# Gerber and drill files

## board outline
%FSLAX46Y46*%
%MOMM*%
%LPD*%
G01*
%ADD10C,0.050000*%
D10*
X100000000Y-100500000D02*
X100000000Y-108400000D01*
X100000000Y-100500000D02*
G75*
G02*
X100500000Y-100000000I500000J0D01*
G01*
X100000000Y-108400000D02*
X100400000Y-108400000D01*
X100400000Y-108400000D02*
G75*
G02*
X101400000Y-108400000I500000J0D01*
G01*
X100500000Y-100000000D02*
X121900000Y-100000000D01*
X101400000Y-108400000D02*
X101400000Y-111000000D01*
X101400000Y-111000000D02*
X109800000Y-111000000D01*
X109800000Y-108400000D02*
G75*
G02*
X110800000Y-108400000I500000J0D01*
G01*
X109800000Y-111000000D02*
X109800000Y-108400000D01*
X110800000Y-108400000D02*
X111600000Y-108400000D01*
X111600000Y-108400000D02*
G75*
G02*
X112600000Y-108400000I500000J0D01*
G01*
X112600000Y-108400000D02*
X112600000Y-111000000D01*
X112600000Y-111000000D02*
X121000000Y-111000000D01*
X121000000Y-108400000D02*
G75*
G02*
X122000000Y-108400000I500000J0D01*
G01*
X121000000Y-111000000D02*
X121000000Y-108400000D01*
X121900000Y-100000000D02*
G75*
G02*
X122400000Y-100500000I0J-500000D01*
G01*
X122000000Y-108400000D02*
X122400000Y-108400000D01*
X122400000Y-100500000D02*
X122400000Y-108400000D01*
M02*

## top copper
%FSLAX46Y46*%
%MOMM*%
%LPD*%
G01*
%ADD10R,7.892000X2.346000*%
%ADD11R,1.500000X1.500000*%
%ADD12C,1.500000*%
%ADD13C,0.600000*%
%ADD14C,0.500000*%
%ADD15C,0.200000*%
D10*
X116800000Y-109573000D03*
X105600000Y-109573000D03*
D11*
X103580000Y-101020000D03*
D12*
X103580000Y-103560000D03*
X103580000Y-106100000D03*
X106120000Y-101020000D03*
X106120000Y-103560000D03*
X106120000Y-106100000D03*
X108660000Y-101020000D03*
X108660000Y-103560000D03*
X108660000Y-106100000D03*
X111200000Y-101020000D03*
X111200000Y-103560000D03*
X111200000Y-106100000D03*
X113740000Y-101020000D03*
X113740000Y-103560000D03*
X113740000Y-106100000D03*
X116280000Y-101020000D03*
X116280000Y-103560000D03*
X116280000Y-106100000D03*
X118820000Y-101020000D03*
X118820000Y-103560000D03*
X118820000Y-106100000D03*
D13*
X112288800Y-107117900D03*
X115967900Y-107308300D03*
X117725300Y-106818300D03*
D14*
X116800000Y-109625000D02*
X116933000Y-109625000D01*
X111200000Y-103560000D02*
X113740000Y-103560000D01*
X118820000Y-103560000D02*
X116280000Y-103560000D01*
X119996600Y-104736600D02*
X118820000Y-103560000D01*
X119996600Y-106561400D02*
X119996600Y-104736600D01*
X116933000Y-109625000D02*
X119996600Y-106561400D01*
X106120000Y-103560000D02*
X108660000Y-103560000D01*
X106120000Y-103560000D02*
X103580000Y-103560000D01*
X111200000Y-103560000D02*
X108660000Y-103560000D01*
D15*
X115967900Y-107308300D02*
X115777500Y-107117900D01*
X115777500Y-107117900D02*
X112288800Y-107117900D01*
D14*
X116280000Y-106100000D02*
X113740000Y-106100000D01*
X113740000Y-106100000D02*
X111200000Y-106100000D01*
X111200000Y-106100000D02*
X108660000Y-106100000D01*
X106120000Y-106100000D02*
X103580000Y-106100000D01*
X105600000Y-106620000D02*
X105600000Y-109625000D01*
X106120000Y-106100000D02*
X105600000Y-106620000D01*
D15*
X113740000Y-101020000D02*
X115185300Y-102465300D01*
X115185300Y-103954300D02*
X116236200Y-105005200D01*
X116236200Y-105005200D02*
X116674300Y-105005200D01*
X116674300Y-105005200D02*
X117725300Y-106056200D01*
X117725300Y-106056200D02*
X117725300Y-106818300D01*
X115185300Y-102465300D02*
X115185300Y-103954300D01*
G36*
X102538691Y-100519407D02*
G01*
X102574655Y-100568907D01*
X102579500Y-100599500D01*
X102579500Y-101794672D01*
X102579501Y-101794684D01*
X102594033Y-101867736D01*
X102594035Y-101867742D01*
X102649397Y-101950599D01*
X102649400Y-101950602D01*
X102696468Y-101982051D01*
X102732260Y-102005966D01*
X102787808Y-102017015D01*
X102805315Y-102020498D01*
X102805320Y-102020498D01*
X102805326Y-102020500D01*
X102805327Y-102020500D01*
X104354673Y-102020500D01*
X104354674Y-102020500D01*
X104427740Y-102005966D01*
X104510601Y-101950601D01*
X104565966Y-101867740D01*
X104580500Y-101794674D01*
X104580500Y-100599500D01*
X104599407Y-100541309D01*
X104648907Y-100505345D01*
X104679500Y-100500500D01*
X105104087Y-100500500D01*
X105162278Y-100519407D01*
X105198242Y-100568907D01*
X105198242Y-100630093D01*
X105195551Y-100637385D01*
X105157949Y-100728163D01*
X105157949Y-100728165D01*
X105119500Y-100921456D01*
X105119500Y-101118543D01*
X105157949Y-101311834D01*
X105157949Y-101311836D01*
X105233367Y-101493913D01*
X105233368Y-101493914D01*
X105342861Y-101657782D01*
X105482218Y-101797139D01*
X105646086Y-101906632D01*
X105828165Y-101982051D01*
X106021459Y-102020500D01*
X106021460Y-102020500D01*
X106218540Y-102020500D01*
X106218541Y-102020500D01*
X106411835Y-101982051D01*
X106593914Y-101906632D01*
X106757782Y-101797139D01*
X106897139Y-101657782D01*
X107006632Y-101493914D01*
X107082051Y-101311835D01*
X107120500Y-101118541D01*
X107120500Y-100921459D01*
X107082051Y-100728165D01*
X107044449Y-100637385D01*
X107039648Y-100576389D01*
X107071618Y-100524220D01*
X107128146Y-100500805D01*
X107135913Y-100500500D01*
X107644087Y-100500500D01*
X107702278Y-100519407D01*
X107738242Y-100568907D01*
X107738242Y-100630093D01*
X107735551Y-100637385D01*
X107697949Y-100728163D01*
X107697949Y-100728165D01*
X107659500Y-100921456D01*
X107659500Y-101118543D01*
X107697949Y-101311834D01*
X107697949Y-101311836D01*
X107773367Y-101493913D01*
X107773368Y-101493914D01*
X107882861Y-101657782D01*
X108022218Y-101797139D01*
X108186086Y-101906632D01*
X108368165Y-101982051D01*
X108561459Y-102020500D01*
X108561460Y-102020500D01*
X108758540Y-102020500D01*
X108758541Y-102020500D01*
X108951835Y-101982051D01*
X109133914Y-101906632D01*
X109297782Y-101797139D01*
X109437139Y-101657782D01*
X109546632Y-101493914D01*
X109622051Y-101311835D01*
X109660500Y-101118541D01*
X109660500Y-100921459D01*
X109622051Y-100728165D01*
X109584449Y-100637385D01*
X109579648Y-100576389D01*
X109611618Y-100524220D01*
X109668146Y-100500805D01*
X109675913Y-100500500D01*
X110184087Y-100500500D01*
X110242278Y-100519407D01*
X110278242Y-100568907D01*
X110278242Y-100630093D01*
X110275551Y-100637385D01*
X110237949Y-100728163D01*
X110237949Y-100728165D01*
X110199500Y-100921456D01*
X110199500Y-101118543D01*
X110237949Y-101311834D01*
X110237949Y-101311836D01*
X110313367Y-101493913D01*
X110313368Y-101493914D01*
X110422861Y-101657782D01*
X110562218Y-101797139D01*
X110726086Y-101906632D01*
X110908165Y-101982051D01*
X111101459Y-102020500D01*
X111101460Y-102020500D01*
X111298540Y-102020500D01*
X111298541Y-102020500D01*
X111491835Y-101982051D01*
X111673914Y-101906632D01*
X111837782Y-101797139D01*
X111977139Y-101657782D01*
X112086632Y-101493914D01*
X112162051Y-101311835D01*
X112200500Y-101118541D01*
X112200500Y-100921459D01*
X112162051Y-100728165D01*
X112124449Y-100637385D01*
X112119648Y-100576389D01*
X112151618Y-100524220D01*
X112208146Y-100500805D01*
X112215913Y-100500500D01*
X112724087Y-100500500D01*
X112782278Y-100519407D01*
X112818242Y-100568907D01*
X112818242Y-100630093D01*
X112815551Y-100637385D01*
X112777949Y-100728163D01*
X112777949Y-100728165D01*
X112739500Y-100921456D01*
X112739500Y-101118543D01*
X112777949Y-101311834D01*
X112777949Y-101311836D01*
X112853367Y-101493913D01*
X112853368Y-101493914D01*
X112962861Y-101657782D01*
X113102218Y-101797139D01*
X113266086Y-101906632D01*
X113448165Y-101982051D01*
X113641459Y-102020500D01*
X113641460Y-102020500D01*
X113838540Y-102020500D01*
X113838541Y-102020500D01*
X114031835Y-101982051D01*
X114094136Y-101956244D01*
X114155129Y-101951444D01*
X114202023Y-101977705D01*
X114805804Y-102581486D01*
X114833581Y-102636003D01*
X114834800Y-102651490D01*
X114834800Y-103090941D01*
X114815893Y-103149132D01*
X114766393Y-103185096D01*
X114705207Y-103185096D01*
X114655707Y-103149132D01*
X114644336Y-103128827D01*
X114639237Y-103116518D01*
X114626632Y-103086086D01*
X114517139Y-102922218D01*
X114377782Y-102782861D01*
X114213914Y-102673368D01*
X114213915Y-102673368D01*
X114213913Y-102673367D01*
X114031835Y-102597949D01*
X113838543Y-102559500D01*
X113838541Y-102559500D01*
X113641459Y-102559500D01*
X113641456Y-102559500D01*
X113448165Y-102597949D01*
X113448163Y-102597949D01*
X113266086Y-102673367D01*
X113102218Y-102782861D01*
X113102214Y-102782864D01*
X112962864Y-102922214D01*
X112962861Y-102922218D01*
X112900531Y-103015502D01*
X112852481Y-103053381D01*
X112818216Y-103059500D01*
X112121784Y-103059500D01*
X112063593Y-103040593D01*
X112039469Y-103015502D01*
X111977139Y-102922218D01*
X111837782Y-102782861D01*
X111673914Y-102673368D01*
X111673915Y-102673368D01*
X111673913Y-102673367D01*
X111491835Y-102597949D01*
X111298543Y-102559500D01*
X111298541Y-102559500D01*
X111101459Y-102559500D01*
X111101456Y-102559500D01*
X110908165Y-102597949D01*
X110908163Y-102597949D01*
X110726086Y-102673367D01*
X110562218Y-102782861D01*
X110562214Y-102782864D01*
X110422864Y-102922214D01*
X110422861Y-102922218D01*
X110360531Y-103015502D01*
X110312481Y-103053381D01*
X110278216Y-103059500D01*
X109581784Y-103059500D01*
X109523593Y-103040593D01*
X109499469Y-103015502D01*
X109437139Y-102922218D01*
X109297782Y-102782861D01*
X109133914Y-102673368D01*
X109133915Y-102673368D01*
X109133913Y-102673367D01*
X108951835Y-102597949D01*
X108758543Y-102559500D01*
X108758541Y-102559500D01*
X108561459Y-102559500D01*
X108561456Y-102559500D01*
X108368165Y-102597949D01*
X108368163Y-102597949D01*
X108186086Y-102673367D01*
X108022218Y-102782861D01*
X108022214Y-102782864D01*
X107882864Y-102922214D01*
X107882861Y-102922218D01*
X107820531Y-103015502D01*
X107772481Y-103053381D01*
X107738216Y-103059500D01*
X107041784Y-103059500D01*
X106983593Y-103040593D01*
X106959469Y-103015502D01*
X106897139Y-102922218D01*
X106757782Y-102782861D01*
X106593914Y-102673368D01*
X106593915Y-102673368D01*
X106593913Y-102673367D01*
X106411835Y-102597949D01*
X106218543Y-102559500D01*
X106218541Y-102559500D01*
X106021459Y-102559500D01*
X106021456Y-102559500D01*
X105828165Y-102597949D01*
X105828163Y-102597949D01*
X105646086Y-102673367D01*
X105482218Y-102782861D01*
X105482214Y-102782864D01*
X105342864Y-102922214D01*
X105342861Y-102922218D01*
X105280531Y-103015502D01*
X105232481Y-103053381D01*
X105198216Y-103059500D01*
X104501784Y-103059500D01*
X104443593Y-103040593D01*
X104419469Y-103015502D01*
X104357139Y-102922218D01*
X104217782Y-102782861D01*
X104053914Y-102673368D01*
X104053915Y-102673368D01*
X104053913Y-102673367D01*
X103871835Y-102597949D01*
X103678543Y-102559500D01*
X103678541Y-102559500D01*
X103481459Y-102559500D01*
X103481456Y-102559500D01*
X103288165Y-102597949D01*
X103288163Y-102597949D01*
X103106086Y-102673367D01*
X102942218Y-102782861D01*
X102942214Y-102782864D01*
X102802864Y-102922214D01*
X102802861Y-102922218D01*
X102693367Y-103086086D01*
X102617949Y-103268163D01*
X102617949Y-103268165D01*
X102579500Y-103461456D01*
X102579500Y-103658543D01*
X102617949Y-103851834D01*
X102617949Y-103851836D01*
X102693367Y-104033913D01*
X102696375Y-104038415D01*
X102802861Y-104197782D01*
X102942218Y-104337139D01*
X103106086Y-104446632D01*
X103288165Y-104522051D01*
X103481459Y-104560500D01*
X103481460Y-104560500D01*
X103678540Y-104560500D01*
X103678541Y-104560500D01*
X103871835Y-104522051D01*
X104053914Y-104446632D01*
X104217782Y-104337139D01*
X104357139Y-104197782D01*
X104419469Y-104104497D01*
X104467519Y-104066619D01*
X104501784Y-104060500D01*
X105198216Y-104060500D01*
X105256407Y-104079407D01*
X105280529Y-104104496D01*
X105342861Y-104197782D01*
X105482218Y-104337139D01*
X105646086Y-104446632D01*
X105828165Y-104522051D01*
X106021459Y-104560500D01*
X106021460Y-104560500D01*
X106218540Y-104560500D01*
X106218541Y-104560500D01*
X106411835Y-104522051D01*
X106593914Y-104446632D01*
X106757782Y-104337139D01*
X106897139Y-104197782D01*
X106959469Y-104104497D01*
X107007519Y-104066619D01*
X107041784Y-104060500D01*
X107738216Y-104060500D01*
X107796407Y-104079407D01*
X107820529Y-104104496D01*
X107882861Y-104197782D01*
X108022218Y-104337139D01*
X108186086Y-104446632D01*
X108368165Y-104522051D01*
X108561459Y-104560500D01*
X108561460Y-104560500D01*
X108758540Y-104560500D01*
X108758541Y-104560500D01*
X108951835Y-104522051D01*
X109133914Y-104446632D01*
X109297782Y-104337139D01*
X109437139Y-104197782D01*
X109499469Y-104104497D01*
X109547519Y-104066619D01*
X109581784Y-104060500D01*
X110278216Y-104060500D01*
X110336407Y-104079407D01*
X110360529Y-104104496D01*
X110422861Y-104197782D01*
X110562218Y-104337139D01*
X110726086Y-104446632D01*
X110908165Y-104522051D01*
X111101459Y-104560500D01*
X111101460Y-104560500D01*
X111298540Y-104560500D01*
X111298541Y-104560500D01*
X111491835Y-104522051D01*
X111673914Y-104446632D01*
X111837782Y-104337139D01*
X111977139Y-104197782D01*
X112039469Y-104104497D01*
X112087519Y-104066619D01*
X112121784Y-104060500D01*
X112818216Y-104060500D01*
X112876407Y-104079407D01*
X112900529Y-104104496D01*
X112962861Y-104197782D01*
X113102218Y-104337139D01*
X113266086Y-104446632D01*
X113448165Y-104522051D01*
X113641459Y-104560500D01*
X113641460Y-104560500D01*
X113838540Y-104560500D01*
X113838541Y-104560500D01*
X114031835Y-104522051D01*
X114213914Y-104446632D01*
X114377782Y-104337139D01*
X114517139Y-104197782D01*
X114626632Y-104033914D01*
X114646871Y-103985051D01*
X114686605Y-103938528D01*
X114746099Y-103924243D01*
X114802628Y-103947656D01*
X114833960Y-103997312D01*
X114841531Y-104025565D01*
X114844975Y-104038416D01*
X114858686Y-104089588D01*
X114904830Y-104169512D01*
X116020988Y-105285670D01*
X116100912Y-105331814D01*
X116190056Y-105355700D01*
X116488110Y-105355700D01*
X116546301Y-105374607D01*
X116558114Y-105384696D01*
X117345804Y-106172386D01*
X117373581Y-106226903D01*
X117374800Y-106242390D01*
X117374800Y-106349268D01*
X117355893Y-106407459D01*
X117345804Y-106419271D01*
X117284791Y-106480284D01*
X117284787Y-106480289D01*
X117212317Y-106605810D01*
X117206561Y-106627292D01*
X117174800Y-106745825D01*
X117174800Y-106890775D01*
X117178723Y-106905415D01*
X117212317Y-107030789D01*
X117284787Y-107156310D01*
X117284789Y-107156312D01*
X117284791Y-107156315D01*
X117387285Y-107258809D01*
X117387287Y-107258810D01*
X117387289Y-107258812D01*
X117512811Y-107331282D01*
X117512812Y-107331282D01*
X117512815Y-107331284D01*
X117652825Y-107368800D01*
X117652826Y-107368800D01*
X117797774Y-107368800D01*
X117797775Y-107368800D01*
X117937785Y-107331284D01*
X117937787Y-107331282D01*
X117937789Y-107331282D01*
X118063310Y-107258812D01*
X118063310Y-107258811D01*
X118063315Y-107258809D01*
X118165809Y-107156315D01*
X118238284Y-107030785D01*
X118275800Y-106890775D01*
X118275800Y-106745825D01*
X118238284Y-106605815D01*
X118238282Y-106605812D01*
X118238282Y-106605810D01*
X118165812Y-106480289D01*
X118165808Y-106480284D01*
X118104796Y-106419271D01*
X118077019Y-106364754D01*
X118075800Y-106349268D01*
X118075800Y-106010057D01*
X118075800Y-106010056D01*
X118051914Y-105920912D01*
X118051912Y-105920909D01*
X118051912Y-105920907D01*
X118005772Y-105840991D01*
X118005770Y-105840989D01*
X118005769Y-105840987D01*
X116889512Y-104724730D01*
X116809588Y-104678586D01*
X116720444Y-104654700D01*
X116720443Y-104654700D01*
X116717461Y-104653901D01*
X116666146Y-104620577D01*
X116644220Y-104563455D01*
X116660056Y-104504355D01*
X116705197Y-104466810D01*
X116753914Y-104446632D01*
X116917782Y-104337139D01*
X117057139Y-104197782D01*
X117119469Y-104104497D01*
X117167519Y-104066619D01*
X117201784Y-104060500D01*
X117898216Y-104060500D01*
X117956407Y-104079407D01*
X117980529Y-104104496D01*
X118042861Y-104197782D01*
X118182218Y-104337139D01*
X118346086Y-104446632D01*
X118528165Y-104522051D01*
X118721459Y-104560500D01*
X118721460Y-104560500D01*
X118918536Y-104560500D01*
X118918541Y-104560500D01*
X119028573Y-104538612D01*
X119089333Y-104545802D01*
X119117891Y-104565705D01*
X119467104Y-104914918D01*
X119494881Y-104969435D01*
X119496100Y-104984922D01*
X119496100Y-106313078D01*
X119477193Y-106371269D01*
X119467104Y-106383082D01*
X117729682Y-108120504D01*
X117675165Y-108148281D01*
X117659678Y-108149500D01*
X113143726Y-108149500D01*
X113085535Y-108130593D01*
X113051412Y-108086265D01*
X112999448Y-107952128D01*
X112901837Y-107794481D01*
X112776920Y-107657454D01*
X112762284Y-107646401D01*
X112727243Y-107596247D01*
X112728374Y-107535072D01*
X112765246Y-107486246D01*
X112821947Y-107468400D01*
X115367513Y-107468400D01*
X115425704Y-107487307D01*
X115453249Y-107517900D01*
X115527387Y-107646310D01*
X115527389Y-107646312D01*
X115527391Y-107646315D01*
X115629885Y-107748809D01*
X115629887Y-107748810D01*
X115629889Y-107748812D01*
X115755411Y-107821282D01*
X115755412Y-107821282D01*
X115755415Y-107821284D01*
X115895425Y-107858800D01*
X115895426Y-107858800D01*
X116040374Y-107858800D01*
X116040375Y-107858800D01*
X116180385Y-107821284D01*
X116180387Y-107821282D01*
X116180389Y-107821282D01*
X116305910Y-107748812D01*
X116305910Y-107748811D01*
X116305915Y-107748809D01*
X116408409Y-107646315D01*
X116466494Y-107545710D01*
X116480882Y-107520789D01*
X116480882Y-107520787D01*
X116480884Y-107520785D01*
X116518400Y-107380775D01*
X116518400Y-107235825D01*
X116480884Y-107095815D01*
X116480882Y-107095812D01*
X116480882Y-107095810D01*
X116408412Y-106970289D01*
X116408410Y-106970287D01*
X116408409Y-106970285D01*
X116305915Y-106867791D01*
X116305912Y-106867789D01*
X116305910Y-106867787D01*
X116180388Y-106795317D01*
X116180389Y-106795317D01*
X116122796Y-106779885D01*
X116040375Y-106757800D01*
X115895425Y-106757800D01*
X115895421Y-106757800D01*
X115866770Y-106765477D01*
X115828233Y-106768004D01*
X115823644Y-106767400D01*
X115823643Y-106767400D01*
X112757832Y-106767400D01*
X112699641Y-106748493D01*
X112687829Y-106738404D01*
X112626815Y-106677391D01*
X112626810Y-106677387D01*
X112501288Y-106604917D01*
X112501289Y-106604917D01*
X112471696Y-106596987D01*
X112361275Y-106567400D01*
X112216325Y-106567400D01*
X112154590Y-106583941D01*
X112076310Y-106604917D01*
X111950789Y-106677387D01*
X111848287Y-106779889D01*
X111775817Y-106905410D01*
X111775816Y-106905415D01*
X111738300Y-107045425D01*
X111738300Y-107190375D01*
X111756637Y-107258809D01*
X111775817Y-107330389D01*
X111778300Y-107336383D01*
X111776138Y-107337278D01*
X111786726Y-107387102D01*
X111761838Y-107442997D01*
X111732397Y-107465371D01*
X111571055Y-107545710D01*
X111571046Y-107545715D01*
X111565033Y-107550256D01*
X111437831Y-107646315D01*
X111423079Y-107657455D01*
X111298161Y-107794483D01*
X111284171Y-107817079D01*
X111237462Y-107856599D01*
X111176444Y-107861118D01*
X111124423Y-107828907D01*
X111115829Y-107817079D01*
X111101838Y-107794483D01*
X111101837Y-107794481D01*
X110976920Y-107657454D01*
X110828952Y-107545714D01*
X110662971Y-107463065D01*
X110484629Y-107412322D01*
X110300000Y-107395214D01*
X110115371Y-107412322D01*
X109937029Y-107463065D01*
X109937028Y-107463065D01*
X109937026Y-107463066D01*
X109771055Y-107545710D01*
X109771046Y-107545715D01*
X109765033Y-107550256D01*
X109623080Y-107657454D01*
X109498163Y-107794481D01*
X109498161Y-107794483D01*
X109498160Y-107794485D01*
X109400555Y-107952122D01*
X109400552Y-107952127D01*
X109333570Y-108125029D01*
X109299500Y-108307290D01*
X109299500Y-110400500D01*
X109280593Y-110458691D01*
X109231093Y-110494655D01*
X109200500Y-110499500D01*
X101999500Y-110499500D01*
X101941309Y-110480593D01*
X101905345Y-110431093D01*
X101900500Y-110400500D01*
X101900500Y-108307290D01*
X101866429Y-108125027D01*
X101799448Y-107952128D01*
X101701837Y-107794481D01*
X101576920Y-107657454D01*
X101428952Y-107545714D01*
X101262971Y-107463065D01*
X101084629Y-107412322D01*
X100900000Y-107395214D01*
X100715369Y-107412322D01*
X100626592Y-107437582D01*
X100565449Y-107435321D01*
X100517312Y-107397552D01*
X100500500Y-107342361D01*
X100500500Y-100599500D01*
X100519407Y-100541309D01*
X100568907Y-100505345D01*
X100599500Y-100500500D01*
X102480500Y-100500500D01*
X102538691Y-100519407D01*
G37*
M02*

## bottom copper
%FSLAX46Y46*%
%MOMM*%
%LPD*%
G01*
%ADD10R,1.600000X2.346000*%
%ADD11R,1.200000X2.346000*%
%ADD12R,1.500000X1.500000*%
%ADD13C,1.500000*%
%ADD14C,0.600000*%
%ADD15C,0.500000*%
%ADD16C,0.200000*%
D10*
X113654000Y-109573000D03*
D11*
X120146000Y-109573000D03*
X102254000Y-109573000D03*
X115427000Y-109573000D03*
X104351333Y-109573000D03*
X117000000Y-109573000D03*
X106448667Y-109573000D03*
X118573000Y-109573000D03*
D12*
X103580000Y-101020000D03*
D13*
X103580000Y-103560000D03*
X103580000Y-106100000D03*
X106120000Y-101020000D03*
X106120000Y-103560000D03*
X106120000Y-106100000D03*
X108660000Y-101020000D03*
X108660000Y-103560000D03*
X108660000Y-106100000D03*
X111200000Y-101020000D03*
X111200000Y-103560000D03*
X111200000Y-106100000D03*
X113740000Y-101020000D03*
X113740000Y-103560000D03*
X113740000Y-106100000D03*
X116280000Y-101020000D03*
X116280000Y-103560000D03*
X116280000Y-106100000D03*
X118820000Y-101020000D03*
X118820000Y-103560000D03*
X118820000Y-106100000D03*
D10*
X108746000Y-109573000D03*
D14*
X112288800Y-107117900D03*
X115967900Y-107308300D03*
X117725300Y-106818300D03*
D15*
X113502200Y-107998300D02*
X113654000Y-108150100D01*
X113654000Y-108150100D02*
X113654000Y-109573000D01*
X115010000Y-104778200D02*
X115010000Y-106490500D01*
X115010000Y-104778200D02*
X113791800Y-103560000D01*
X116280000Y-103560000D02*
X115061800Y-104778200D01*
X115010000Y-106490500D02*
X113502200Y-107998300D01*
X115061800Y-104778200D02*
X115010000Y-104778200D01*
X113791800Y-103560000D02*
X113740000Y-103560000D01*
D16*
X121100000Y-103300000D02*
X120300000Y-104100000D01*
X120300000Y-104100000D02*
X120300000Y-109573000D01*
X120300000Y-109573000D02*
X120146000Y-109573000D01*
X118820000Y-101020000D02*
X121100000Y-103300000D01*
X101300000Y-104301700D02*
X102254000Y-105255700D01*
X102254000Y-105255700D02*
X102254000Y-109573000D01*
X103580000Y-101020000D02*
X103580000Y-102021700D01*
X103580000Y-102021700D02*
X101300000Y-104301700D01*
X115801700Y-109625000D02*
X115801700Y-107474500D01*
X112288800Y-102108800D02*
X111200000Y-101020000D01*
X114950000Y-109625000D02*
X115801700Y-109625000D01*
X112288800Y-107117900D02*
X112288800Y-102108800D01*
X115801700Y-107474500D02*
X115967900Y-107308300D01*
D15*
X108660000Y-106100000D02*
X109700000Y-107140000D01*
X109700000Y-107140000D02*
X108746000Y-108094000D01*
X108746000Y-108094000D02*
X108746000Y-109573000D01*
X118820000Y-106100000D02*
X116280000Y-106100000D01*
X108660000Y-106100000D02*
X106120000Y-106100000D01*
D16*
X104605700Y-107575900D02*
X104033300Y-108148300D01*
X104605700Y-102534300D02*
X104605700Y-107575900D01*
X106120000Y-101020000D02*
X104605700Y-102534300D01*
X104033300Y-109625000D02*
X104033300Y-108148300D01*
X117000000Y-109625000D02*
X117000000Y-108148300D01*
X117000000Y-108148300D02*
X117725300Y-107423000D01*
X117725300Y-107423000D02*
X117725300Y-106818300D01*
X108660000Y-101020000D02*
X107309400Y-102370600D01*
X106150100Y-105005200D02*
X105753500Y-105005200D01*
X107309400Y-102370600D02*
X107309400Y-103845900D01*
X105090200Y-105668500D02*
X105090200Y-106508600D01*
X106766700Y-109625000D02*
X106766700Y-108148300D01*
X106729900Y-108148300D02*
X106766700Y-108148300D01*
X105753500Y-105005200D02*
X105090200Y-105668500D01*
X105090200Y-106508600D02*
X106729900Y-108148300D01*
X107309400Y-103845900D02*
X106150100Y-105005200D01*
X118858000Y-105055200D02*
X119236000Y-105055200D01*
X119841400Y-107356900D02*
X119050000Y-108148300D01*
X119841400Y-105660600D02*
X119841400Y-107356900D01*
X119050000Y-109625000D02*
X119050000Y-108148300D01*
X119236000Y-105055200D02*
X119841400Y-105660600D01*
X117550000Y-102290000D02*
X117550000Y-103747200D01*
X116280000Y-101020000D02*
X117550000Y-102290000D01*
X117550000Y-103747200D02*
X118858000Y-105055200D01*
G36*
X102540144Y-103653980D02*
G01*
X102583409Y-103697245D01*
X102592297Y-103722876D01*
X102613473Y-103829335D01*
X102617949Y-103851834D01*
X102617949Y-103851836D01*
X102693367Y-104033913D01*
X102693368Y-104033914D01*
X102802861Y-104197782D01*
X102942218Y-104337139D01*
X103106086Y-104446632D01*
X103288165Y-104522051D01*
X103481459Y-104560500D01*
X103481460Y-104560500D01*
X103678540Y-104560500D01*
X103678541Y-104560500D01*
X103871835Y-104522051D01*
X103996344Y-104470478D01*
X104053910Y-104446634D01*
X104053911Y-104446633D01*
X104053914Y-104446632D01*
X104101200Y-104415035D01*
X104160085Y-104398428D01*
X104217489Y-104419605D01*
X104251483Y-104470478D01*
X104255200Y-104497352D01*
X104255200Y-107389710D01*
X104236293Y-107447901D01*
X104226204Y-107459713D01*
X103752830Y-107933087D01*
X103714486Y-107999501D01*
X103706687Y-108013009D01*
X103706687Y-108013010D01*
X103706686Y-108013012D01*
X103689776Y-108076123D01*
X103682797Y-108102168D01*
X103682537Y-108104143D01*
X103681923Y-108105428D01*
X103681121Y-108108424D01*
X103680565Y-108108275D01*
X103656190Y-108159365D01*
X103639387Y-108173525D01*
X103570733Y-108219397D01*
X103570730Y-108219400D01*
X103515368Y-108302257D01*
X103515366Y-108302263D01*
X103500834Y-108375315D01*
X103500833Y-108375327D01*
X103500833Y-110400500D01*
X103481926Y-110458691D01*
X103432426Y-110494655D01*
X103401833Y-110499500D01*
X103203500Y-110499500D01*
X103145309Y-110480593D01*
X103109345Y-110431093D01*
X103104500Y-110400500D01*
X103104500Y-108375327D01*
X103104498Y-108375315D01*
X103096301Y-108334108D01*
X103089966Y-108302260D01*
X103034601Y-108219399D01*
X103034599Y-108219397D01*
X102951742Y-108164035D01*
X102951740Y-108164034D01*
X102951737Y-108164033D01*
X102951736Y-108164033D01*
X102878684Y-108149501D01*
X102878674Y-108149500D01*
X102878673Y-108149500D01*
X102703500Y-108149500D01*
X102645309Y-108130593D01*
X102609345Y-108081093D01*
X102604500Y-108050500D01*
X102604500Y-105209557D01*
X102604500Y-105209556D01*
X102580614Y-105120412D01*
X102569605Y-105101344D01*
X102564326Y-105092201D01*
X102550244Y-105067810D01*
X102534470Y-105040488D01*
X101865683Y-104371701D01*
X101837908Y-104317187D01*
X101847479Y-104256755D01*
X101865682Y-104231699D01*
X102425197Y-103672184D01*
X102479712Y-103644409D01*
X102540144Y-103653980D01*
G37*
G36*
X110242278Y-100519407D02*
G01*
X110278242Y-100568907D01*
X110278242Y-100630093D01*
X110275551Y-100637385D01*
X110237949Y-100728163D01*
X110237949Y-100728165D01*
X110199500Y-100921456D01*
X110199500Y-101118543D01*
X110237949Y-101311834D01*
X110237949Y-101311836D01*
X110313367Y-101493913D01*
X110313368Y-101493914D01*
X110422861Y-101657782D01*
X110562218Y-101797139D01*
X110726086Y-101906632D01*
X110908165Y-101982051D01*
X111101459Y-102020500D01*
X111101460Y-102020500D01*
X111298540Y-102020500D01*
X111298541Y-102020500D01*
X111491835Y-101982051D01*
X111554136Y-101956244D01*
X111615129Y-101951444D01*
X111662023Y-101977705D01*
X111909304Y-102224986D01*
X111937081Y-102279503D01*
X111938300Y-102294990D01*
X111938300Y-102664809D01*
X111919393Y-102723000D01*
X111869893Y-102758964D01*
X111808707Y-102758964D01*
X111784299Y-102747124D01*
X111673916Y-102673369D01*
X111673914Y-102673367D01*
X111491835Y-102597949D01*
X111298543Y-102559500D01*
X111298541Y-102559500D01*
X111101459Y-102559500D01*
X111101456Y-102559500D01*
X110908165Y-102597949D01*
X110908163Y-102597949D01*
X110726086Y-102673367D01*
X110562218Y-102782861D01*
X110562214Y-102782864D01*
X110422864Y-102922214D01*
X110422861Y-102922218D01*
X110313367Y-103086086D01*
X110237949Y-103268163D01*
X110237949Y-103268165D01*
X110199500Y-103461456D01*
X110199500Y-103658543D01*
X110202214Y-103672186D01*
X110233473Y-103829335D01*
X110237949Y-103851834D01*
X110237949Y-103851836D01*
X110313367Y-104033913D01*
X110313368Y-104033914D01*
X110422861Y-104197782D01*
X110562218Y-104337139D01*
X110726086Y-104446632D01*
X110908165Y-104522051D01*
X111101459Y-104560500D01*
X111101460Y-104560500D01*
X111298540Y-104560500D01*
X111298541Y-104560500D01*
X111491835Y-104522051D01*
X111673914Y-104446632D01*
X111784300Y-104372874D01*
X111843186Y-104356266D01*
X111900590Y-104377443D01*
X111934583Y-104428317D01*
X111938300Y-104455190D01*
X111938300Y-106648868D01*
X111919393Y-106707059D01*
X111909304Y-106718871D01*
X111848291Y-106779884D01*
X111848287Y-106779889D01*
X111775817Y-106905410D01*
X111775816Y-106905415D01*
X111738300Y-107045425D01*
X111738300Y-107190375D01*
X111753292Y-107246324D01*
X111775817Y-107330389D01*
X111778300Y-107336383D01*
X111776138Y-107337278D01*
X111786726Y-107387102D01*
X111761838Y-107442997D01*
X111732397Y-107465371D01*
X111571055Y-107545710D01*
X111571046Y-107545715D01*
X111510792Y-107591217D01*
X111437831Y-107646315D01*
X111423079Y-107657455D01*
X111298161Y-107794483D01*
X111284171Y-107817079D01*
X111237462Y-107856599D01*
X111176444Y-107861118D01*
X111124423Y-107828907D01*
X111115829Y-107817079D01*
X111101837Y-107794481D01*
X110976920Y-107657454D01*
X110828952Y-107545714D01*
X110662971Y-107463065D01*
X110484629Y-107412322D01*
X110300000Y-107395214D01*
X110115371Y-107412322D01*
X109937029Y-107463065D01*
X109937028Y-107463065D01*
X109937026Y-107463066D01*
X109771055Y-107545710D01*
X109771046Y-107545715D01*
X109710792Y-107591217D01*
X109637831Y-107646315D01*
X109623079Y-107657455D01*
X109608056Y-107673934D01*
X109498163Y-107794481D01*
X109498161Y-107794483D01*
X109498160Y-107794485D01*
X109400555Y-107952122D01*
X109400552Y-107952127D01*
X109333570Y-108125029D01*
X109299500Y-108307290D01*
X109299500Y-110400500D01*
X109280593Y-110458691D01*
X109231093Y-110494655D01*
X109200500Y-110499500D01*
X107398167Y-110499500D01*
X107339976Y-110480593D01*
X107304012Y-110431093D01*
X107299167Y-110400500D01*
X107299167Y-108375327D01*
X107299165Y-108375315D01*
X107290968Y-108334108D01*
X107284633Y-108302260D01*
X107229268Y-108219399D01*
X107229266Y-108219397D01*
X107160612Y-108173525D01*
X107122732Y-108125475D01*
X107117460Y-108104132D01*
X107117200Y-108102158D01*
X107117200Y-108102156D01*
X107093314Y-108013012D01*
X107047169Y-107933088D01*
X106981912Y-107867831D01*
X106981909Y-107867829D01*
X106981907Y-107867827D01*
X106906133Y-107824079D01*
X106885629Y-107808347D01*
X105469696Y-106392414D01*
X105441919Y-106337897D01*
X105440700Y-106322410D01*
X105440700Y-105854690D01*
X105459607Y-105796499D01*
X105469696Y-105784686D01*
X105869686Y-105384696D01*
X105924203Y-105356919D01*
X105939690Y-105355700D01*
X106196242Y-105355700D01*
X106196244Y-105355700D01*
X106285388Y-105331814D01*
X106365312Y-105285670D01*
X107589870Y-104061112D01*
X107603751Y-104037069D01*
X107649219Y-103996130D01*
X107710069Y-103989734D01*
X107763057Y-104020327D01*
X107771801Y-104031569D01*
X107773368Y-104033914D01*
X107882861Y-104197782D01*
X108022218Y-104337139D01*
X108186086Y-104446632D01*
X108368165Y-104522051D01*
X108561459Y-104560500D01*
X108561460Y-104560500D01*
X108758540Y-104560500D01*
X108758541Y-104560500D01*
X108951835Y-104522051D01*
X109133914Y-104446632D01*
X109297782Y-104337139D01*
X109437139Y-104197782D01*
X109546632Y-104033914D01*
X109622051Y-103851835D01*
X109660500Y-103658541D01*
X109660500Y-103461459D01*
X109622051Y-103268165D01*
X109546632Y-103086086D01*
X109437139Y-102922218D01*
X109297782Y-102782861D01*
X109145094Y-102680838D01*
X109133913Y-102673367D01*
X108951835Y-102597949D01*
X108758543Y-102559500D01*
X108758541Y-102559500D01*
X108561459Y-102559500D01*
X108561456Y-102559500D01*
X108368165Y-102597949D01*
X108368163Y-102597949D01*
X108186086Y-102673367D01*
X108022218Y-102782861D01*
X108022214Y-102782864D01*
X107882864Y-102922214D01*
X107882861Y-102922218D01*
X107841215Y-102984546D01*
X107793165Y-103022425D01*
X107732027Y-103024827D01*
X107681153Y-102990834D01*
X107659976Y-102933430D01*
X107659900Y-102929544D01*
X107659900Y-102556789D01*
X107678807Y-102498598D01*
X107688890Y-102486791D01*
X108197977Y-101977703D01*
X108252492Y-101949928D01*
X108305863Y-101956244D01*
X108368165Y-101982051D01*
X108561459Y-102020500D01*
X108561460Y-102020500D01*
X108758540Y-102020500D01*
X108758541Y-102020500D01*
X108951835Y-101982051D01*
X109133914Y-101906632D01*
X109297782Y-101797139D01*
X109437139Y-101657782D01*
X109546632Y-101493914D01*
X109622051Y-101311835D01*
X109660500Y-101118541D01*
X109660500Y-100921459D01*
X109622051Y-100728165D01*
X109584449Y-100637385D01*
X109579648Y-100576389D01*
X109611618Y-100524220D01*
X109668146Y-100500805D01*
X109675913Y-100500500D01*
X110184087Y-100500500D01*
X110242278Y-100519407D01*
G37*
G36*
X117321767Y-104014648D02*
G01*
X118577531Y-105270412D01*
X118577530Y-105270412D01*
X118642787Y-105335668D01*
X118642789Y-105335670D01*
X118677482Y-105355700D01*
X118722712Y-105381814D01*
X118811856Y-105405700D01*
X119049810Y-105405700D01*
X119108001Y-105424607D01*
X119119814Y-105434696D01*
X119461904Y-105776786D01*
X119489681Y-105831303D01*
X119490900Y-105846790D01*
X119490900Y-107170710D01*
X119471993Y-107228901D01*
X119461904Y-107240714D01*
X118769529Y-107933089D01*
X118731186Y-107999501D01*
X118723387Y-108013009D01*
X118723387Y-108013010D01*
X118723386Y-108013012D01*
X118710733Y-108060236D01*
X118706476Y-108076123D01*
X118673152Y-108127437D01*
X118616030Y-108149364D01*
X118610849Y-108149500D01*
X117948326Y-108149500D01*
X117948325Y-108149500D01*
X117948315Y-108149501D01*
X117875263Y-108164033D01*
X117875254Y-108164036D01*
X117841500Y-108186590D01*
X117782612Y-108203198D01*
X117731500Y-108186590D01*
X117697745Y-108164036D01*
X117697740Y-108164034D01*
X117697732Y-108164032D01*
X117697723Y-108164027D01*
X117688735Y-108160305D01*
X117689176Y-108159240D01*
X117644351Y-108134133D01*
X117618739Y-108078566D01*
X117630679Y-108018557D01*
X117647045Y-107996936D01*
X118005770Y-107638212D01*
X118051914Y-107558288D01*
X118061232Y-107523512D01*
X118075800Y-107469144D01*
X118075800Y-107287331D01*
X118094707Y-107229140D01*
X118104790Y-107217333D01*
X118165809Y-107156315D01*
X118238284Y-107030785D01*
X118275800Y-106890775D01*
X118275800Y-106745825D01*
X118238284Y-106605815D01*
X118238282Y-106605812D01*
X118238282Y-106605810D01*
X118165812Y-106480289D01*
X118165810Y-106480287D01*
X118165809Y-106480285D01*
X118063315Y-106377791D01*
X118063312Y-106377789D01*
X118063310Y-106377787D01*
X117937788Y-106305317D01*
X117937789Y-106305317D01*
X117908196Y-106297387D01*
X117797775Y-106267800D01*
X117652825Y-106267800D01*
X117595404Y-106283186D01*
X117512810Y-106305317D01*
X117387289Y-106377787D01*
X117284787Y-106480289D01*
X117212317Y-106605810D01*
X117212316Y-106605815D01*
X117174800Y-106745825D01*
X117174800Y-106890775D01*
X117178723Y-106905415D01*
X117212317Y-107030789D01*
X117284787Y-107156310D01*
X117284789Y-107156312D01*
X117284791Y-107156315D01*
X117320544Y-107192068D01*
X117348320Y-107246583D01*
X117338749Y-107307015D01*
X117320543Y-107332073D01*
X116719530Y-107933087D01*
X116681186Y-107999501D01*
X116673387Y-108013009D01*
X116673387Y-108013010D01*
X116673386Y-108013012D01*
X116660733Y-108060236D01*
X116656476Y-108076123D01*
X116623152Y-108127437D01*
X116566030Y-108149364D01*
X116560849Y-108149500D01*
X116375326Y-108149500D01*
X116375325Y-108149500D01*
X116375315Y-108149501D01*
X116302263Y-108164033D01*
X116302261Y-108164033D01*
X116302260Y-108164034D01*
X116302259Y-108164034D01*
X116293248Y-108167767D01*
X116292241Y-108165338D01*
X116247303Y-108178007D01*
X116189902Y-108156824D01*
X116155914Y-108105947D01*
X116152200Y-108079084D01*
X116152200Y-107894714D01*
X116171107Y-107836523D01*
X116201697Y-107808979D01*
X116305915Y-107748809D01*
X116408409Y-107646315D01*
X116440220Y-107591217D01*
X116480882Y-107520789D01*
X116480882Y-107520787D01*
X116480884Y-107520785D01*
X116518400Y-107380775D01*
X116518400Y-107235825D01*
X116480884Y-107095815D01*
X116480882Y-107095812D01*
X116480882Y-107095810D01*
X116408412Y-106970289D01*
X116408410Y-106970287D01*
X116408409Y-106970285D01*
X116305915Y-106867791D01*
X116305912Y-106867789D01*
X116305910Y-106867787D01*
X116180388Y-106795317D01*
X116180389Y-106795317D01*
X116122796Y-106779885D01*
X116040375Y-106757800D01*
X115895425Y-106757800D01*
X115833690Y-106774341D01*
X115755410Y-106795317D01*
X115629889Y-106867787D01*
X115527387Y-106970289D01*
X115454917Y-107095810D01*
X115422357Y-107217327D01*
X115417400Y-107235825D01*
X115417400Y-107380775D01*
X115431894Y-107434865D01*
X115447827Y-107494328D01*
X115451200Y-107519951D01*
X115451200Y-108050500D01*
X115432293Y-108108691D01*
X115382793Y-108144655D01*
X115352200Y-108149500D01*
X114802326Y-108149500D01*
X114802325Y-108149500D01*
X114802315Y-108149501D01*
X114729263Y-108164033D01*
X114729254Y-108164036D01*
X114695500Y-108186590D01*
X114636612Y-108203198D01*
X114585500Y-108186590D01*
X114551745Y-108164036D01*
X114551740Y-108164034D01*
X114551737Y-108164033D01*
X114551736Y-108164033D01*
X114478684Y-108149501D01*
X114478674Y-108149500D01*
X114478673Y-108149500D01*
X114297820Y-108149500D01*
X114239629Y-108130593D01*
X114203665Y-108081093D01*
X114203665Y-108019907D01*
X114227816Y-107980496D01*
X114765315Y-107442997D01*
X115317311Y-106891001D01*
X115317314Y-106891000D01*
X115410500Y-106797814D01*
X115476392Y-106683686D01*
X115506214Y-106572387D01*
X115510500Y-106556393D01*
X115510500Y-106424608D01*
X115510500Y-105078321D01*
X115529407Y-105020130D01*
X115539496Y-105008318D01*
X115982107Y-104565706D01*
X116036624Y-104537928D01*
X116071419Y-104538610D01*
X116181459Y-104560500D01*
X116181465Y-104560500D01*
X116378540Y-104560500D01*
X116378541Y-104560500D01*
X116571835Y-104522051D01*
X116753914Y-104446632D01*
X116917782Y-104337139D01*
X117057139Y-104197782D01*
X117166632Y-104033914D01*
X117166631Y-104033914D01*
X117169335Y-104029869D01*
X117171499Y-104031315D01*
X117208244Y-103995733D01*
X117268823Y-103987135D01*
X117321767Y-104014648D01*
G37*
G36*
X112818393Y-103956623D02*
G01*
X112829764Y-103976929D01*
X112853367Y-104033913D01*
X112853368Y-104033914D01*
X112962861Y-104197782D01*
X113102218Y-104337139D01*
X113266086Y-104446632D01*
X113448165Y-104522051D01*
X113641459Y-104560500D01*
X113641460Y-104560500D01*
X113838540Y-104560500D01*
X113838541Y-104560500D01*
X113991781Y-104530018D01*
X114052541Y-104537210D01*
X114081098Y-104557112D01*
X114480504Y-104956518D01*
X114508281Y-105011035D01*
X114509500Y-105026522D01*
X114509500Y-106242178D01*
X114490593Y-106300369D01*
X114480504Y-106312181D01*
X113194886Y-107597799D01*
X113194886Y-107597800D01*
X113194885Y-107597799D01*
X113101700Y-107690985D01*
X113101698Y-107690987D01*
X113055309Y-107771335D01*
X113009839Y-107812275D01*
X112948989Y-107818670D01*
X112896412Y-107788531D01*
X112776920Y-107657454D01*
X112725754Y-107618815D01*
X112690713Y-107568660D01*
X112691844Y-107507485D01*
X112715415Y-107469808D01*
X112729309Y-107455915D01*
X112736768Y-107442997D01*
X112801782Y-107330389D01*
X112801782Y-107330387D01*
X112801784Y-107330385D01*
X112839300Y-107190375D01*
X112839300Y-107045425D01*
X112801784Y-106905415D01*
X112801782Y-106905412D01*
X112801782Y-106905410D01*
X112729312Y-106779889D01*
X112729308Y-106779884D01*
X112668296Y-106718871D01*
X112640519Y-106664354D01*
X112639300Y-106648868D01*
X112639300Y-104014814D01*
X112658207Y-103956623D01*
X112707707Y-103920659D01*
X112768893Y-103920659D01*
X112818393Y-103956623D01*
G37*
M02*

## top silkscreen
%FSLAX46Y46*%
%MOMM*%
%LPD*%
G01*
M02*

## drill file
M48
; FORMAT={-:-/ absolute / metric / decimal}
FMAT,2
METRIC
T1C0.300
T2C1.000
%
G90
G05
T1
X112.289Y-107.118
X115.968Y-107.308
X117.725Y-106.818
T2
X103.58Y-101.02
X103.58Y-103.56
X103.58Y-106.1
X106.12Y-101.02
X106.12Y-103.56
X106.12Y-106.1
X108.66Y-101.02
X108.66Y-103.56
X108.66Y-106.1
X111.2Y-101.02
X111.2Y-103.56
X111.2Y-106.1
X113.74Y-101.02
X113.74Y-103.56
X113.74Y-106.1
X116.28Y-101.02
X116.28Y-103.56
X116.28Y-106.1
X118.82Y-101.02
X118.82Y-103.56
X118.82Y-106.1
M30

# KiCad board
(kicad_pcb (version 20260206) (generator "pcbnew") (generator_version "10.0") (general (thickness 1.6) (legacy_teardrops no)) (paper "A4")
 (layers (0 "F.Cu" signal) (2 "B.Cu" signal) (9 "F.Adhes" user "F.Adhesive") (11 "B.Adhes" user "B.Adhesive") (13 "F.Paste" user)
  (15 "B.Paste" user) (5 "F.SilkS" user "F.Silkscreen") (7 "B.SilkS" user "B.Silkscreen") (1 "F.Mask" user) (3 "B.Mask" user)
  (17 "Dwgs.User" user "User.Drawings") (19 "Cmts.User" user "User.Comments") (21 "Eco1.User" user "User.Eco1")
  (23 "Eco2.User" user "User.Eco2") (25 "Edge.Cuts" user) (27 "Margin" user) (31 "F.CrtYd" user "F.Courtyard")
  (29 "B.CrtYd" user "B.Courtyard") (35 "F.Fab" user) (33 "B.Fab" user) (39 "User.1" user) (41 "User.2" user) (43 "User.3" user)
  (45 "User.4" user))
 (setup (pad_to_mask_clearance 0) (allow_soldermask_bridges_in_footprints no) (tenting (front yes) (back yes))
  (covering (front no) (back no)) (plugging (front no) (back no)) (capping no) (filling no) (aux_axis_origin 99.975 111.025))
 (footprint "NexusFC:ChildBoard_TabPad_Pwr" (layer "F.Cu") (at 113.654 108.4)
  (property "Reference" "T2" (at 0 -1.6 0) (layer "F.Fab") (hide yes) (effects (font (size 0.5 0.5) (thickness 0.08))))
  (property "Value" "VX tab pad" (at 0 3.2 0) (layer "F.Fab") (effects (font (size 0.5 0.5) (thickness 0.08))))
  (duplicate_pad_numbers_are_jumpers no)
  (pad "1" smd rect (at 0 1.173) (size 1.6 2.346) (layers "B.Cu" "B.Mask") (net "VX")))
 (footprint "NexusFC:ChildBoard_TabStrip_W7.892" (layer "F.Cu") (at 116.8 108.4)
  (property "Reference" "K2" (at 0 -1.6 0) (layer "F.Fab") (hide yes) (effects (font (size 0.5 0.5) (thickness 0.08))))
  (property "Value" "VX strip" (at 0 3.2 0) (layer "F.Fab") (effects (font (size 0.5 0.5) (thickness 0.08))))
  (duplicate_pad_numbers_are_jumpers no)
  (pad "1" smd rect (at 0 1.173) (size 7.892 2.346) (layers "F.Cu" "F.Mask") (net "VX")))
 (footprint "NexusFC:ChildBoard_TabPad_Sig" (layer "F.Cu") (at 120.146 108.4)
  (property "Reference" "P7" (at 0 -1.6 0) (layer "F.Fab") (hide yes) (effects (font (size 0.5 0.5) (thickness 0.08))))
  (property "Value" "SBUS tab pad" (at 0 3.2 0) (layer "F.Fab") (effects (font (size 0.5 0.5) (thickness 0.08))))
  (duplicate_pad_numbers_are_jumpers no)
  (pad "1" smd rect (at 0 1.173) (size 1.2 2.346) (layers "B.Cu" "B.Mask") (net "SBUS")))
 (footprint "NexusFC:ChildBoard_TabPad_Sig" (layer "F.Cu") (at 102.254 108.4)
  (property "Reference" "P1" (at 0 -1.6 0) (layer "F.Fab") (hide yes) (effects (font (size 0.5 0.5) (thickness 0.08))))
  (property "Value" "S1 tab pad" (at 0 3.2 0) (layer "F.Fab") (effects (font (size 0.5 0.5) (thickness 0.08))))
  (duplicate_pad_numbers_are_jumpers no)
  (pad "1" smd rect (at 0 1.173) (size 1.2 2.346) (layers "B.Cu" "B.Mask") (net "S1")))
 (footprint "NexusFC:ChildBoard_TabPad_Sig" (layer "F.Cu") (at 115.427 108.4)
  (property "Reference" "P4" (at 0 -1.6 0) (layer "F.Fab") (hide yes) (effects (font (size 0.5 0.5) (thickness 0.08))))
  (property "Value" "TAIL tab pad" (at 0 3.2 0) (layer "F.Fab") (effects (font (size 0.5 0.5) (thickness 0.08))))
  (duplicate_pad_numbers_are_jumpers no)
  (pad "1" smd rect (at 0 1.173) (size 1.2 2.346) (layers "B.Cu" "B.Mask") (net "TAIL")))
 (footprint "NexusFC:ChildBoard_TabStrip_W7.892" (layer "F.Cu") (at 105.6 108.4)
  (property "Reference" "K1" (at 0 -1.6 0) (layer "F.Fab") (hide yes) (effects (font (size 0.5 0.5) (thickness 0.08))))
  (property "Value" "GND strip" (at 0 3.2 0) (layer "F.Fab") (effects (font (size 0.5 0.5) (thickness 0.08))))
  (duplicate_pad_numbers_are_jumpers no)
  (pad "1" smd rect (at 0 1.173) (size 7.892 2.346) (layers "F.Cu" "F.Mask") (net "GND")))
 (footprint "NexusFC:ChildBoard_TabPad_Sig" (layer "F.Cu") (at 104.351333 108.4)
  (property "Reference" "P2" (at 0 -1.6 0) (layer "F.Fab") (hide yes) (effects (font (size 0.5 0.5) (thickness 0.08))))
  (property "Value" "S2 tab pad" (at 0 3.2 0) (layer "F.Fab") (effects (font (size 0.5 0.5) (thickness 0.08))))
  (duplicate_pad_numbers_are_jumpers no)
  (pad "1" smd rect (at 0 1.173) (size 1.2 2.346) (layers "B.Cu" "B.Mask") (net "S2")))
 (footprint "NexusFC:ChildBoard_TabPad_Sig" (layer "F.Cu") (at 117 108.4)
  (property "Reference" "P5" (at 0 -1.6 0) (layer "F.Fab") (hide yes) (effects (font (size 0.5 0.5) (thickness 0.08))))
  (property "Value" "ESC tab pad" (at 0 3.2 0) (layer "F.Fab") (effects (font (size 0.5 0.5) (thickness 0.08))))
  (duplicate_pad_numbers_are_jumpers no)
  (pad "1" smd rect (at 0 1.173) (size 1.2 2.346) (layers "B.Cu" "B.Mask") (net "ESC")))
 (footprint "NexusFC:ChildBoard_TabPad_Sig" (layer "F.Cu") (at 106.448667 108.4)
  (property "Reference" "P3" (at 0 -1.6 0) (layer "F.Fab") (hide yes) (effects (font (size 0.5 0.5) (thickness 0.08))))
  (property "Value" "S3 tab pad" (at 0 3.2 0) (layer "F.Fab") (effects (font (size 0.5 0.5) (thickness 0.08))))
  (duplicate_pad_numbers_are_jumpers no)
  (pad "1" smd rect (at 0 1.173) (size 1.2 2.346) (layers "B.Cu" "B.Mask") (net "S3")))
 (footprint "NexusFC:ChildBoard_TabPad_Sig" (layer "F.Cu") (at 118.573 108.4)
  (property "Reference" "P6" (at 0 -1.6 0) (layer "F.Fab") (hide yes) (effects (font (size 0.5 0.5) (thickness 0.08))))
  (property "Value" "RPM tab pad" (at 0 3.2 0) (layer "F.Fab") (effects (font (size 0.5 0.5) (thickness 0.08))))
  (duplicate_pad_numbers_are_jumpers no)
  (pad "1" smd rect (at 0 1.173) (size 1.2 2.346) (layers "B.Cu" "B.Mask") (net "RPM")))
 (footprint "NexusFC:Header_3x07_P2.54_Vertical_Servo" (layer "F.Cu") (at 111.2 103.56)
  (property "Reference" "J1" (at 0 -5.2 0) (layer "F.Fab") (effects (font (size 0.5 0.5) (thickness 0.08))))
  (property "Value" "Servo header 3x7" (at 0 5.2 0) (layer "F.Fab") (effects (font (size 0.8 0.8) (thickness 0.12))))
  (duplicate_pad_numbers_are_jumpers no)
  (pad "1" thru_hole rect (at -7.62 -2.54) (size 1.5 1.5) (drill 1) (layers "*.Cu" "*.Mask") (remove_unused_layers no) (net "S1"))
  (pad "2" thru_hole circle (at -7.62 0) (size 1.5 1.5) (drill 1) (layers "*.Cu" "*.Mask") (remove_unused_layers no) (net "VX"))
  (pad "3" thru_hole circle (at -7.62 2.54) (size 1.5 1.5) (drill 1) (layers "*.Cu" "*.Mask") (remove_unused_layers no) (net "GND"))
  (pad "4" thru_hole circle (at -5.08 -2.54) (size 1.5 1.5) (drill 1) (layers "*.Cu" "*.Mask") (remove_unused_layers no) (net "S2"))
  (pad "5" thru_hole circle (at -5.08 0) (size 1.5 1.5) (drill 1) (layers "*.Cu" "*.Mask") (remove_unused_layers no) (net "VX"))
  (pad "6" thru_hole circle (at -5.08 2.54) (size 1.5 1.5) (drill 1) (layers "*.Cu" "*.Mask") (remove_unused_layers no) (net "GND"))
  (pad "7" thru_hole circle (at -2.54 -2.54) (size 1.5 1.5) (drill 1) (layers "*.Cu" "*.Mask") (remove_unused_layers no) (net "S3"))
  (pad "8" thru_hole circle (at -2.54 0) (size 1.5 1.5) (drill 1) (layers "*.Cu" "*.Mask") (remove_unused_layers no) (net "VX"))
  (pad "9" thru_hole circle (at -2.54 2.54) (size 1.5 1.5) (drill 1) (layers "*.Cu" "*.Mask") (remove_unused_layers no) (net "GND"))
  (pad "10" thru_hole circle (at 0 -2.54) (size 1.5 1.5) (drill 1) (layers "*.Cu" "*.Mask") (remove_unused_layers no) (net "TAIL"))
  (pad "11" thru_hole circle (at 0 0) (size 1.5 1.5) (drill 1) (layers "*.Cu" "*.Mask") (remove_unused_layers no) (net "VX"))
  (pad "12" thru_hole circle (at 0 2.54) (size 1.5 1.5) (drill 1) (layers "*.Cu" "*.Mask") (remove_unused_layers no) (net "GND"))
  (pad "13" thru_hole circle (at 2.54 -2.54) (size 1.5 1.5) (drill 1) (layers "*.Cu" "*.Mask") (remove_unused_layers no) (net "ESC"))
  (pad "14" thru_hole circle (at 2.54 0) (size 1.5 1.5) (drill 1) (layers "*.Cu" "*.Mask") (remove_unused_layers no) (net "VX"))
  (pad "15" thru_hole circle (at 2.54 2.54) (size 1.5 1.5) (drill 1) (layers "*.Cu" "*.Mask") (remove_unused_layers no) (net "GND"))
  (pad "16" thru_hole circle (at 5.08 -2.54) (size 1.5 1.5) (drill 1) (layers "*.Cu" "*.Mask") (remove_unused_layers no) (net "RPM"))
  (pad "17" thru_hole circle (at 5.08 0) (size 1.5 1.5) (drill 1) (layers "*.Cu" "*.Mask") (remove_unused_layers no) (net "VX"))
  (pad "18" thru_hole circle (at 5.08 2.54) (size 1.5 1.5) (drill 1) (layers "*.Cu" "*.Mask") (remove_unused_layers no) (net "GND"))
  (pad "19" thru_hole circle (at 7.62 -2.54) (size 1.5 1.5) (drill 1) (layers "*.Cu" "*.Mask") (remove_unused_layers no) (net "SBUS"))
  (pad "20" thru_hole circle (at 7.62 0) (size 1.5 1.5) (drill 1) (layers "*.Cu" "*.Mask") (remove_unused_layers no) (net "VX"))
  (pad "21" thru_hole circle (at 7.62 2.54) (size 1.5 1.5) (drill 1) (layers "*.Cu" "*.Mask") (remove_unused_layers no) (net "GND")))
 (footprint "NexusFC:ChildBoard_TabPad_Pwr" (layer "F.Cu") (at 108.746 108.4)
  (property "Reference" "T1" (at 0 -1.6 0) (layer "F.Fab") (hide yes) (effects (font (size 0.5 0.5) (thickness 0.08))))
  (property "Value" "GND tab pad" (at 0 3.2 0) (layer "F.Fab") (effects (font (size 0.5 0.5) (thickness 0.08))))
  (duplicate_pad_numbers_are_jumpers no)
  (pad "1" smd rect (at 0 1.173) (size 1.6 2.346) (layers "B.Cu" "B.Mask") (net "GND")))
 (gr_line (start 100 100.5) (end 100 108.4) (stroke (width 0.05) (type default)) (layer "Edge.Cuts"))
 (gr_arc (start 100 100.5) (mid 100.146447 100.146447) (end 100.5 100) (stroke (width 0.05) (type default)) (layer "Edge.Cuts"))
 (gr_line (start 100 108.4) (end 100.4 108.4) (stroke (width 0.05) (type solid)) (layer "Edge.Cuts"))
 (gr_arc (start 100.4 108.4) (mid 100.9 107.9) (end 101.4 108.4) (stroke (width 0.05) (type solid)) (layer "Edge.Cuts"))
 (gr_line (start 100.5 100) (end 121.9 100) (stroke (width 0.05) (type default)) (layer "Edge.Cuts"))
 (gr_line (start 101.4 108.4) (end 101.4 111) (stroke (width 0.05) (type solid)) (layer "Edge.Cuts"))
 (gr_line (start 101.4 111) (end 109.8 111) (stroke (width 0.05) (type solid)) (layer "Edge.Cuts"))
 (gr_arc (start 109.8 108.4) (mid 110.3 107.9) (end 110.8 108.4) (stroke (width 0.05) (type solid)) (layer "Edge.Cuts"))
 (gr_line (start 109.8 111) (end 109.8 108.4) (stroke (width 0.05) (type solid)) (layer "Edge.Cuts"))
 (gr_line (start 110.8 108.4) (end 111.6 108.4) (stroke (width 0.05) (type solid)) (layer "Edge.Cuts"))
 (gr_arc (start 111.6 108.4) (mid 112.1 107.9) (end 112.6 108.4) (stroke (width 0.05) (type solid)) (layer "Edge.Cuts"))
 (gr_line (start 112.6 108.4) (end 112.6 111) (stroke (width 0.05) (type solid)) (layer "Edge.Cuts"))
 (gr_line (start 112.6 111) (end 121 111) (stroke (width 0.05) (type solid)) (layer "Edge.Cuts"))
 (gr_arc (start 121 108.4) (mid 121.5 107.9) (end 122 108.4) (stroke (width 0.05) (type solid)) (layer "Edge.Cuts"))
 (gr_line (start 121 111) (end 121 108.4) (stroke (width 0.05) (type solid)) (layer "Edge.Cuts"))
 (gr_arc (start 121.9 100) (mid 122.253553 100.146447) (end 122.4 100.5) (stroke (width 0.05) (type default)) (layer "Edge.Cuts"))
 (gr_line (start 122 108.4) (end 122.4 108.4) (stroke (width 0.05) (type solid)) (layer "Edge.Cuts"))
 (gr_line (start 122.4 100.5) (end 122.4 108.4) (stroke (width 0.05) (type default)) (layer "Edge.Cuts"))
 (segment (start 116.8 109.625) (end 116.933 109.625) (width 0.5) (layer "F.Cu") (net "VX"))
 (segment (start 111.2 103.56) (end 113.74 103.56) (width 0.5) (layer "F.Cu") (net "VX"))
 (segment (start 118.82 103.56) (end 116.28 103.56) (width 0.5) (layer "F.Cu") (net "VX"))
 (segment (start 119.9966 104.7366) (end 118.82 103.56) (width 0.5) (layer "F.Cu") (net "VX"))
 (segment (start 119.9966 106.5614) (end 119.9966 104.7366) (width 0.5) (layer "F.Cu") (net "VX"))
 (segment (start 116.933 109.625) (end 119.9966 106.5614) (width 0.5) (layer "F.Cu") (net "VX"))
 (segment (start 106.12 103.56) (end 108.66 103.56) (width 0.5) (layer "F.Cu") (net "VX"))
 (segment (start 106.12 103.56) (end 103.58 103.56) (width 0.5) (layer "F.Cu") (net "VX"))
 (segment (start 111.2 103.56) (end 108.66 103.56) (width 0.5) (layer "F.Cu") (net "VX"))
 (segment (start 113.5022 107.9983) (end 113.654 108.1501) (width 0.5) (layer "B.Cu") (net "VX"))
 (segment (start 113.654 108.1501) (end 113.654 109.573) (width 0.5) (layer "B.Cu") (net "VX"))
 (segment (start 115.01 104.7782) (end 115.01 106.4905) (width 0.5) (layer "B.Cu") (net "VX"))
 (segment (start 115.01 104.7782) (end 113.7918 103.56) (width 0.5) (layer "B.Cu") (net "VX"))
 (segment (start 116.28 103.56) (end 115.0618 104.7782) (width 0.5) (layer "B.Cu") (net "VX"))
 (segment (start 115.01 106.4905) (end 113.5022 107.9983) (width 0.5) (layer "B.Cu") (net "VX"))
 (segment (start 115.0618 104.7782) (end 115.01 104.7782) (width 0.5) (layer "B.Cu") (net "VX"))
 (segment (start 113.7918 103.56) (end 113.74 103.56) (width 0.5) (layer "B.Cu") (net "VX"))
 (segment (start 121.1 103.3) (end 120.3 104.1) (width 0.2) (layer "B.Cu") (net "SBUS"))
 (segment (start 120.3 104.1) (end 120.3 109.573) (width 0.2) (layer "B.Cu") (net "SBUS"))
 (segment (start 120.3 109.573) (end 120.146 109.573) (width 0.2) (layer "B.Cu") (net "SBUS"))
 (segment (start 118.82 101.02) (end 121.1 103.3) (width 0.2) (layer "B.Cu") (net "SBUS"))
 (segment (start 101.3 104.3017) (end 102.254 105.2557) (width 0.2) (layer "B.Cu") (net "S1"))
 (segment (start 102.254 105.2557) (end 102.254 109.573) (width 0.2) (layer "B.Cu") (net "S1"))
 (segment (start 103.58 101.02) (end 103.58 102.0217) (width 0.2) (layer "B.Cu") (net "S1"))
 (segment (start 103.58 102.0217) (end 101.3 104.3017) (width 0.2) (layer "B.Cu") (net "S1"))
 (segment (start 115.9679 107.3083) (end 115.7775 107.1179) (width 0.2) (layer "F.Cu") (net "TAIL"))
 (segment (start 115.7775 107.1179) (end 112.2888 107.1179) (width 0.2) (layer "F.Cu") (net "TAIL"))
 (via (at 112.2888 107.1179) (size 0.6) (drill 0.3) (layers "F.Cu" "B.Cu") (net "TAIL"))
 (via (at 115.9679 107.3083) (size 0.6) (drill 0.3) (layers "F.Cu" "B.Cu") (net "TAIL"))
 (segment (start 115.8017 109.625) (end 115.8017 107.4745) (width 0.2) (layer "B.Cu") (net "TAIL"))
 (segment (start 112.2888 102.1088) (end 111.2 101.02) (width 0.2) (layer "B.Cu") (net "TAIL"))
 (segment (start 114.95 109.625) (end 115.8017 109.625) (width 0.2) (layer "B.Cu") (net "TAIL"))
 (segment (start 112.2888 107.1179) (end 112.2888 102.1088) (width 0.2) (layer "B.Cu") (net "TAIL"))
 (segment (start 115.8017 107.4745) (end 115.9679 107.3083) (width 0.2) (layer "B.Cu") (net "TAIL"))
 (segment (start 116.28 106.1) (end 113.74 106.1) (width 0.5) (layer "F.Cu") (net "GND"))
 (segment (start 113.74 106.1) (end 111.2 106.1) (width 0.5) (layer "F.Cu") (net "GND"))
 (segment (start 111.2 106.1) (end 108.66 106.1) (width 0.5) (layer "F.Cu") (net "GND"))
 (segment (start 106.12 106.1) (end 103.58 106.1) (width 0.5) (layer "F.Cu") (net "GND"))
 (segment (start 105.6 106.62) (end 105.6 109.625) (width 0.5) (layer "F.Cu") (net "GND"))
 (segment (start 106.12 106.1) (end 105.6 106.62) (width 0.5) (layer "F.Cu") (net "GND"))
 (segment (start 108.66 106.1) (end 109.7 107.14) (width 0.5) (layer "B.Cu") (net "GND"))
 (segment (start 109.7 107.14) (end 108.746 108.094) (width 0.5) (layer "B.Cu") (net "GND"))
 (segment (start 108.746 108.094) (end 108.746 109.573) (width 0.5) (layer "B.Cu") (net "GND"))
 (segment (start 118.82 106.1) (end 116.28 106.1) (width 0.5) (layer "B.Cu") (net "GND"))
 (segment (start 108.66 106.1) (end 106.12 106.1) (width 0.5) (layer "B.Cu") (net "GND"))
 (segment (start 104.6057 107.5759) (end 104.0333 108.1483) (width 0.2) (layer "B.Cu") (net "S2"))
 (segment (start 104.6057 102.5343) (end 104.6057 107.5759) (width 0.2) (layer "B.Cu") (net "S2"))
 (segment (start 106.12 101.02) (end 104.6057 102.5343) (width 0.2) (layer "B.Cu") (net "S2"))
 (segment (start 104.0333 109.625) (end 104.0333 108.1483) (width 0.2) (layer "B.Cu") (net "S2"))
 (segment (start 113.74 101.02) (end 115.1853 102.4653) (width 0.2) (layer "F.Cu") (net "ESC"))
 (segment (start 115.1853 103.9543) (end 116.2362 105.0052) (width 0.2) (layer "F.Cu") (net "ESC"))
 (segment (start 116.2362 105.0052) (end 116.6743 105.0052) (width 0.2) (layer "F.Cu") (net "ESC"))
 (segment (start 116.6743 105.0052) (end 117.7253 106.0562) (width 0.2) (layer "F.Cu") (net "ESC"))
 (segment (start 117.7253 106.0562) (end 117.7253 106.8183) (width 0.2) (layer "F.Cu") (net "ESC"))
 (segment (start 115.1853 102.4653) (end 115.1853 103.9543) (width 0.2) (layer "F.Cu") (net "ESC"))
 (via (at 117.7253 106.8183) (size 0.6) (drill 0.3) (layers "F.Cu" "B.Cu") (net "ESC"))
 (segment (start 117 109.625) (end 117 108.1483) (width 0.2) (layer "B.Cu") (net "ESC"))
 (segment (start 117 108.1483) (end 117.7253 107.423) (width 0.2) (layer "B.Cu") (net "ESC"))
 (segment (start 117.7253 107.423) (end 117.7253 106.8183) (width 0.2) (layer "B.Cu") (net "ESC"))
 (segment (start 108.66 101.02) (end 107.3094 102.3706) (width 0.2) (layer "B.Cu") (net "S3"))
 (segment (start 106.1501 105.0052) (end 105.7535 105.0052) (width 0.2) (layer "B.Cu") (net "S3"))
 (segment (start 107.3094 102.3706) (end 107.3094 103.8459) (width 0.2) (layer "B.Cu") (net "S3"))
 (segment (start 105.0902 105.6685) (end 105.0902 106.5086) (width 0.2) (layer "B.Cu") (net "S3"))
 (segment (start 106.7667 109.625) (end 106.7667 108.1483) (width 0.2) (layer "B.Cu") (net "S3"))
 (segment (start 106.7299 108.1483) (end 106.7667 108.1483) (width 0.2) (layer "B.Cu") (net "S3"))
 (segment (start 105.7535 105.0052) (end 105.0902 105.6685) (width 0.2) (layer "B.Cu") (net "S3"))
 (segment (start 105.0902 106.5086) (end 106.7299 108.1483) (width 0.2) (layer "B.Cu") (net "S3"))
 (segment (start 107.3094 103.8459) (end 106.1501 105.0052) (width 0.2) (layer "B.Cu") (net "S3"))
 (segment (start 118.858 105.0552) (end 119.236 105.0552) (width 0.2) (layer "B.Cu") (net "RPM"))
 (segment (start 119.8414 107.3569) (end 119.05 108.1483) (width 0.2) (layer "B.Cu") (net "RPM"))
 (segment (start 119.8414 105.6606) (end 119.8414 107.3569) (width 0.2) (layer "B.Cu") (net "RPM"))
 (segment (start 119.05 109.625) (end 119.05 108.1483) (width 0.2) (layer "B.Cu") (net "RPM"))
 (segment (start 119.236 105.0552) (end 119.8414 105.6606) (width 0.2) (layer "B.Cu") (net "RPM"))
 (segment (start 117.55 102.29) (end 117.55 103.7472) (width 0.2) (layer "B.Cu") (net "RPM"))
 (segment (start 116.28 101.02) (end 117.55 102.29) (width 0.2) (layer "B.Cu") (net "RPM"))
 (segment (start 117.55 103.7472) (end 118.858 105.0552) (width 0.2) (layer "B.Cu") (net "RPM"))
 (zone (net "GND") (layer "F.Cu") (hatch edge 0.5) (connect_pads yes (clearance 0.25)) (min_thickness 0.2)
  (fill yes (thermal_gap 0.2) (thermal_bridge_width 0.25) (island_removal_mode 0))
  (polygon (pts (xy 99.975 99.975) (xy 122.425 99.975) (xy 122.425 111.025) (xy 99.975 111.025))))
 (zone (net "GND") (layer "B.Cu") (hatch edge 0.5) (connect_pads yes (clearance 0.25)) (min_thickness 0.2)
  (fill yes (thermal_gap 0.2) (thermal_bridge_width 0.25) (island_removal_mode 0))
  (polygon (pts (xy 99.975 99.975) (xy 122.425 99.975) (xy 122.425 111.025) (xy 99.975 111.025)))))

